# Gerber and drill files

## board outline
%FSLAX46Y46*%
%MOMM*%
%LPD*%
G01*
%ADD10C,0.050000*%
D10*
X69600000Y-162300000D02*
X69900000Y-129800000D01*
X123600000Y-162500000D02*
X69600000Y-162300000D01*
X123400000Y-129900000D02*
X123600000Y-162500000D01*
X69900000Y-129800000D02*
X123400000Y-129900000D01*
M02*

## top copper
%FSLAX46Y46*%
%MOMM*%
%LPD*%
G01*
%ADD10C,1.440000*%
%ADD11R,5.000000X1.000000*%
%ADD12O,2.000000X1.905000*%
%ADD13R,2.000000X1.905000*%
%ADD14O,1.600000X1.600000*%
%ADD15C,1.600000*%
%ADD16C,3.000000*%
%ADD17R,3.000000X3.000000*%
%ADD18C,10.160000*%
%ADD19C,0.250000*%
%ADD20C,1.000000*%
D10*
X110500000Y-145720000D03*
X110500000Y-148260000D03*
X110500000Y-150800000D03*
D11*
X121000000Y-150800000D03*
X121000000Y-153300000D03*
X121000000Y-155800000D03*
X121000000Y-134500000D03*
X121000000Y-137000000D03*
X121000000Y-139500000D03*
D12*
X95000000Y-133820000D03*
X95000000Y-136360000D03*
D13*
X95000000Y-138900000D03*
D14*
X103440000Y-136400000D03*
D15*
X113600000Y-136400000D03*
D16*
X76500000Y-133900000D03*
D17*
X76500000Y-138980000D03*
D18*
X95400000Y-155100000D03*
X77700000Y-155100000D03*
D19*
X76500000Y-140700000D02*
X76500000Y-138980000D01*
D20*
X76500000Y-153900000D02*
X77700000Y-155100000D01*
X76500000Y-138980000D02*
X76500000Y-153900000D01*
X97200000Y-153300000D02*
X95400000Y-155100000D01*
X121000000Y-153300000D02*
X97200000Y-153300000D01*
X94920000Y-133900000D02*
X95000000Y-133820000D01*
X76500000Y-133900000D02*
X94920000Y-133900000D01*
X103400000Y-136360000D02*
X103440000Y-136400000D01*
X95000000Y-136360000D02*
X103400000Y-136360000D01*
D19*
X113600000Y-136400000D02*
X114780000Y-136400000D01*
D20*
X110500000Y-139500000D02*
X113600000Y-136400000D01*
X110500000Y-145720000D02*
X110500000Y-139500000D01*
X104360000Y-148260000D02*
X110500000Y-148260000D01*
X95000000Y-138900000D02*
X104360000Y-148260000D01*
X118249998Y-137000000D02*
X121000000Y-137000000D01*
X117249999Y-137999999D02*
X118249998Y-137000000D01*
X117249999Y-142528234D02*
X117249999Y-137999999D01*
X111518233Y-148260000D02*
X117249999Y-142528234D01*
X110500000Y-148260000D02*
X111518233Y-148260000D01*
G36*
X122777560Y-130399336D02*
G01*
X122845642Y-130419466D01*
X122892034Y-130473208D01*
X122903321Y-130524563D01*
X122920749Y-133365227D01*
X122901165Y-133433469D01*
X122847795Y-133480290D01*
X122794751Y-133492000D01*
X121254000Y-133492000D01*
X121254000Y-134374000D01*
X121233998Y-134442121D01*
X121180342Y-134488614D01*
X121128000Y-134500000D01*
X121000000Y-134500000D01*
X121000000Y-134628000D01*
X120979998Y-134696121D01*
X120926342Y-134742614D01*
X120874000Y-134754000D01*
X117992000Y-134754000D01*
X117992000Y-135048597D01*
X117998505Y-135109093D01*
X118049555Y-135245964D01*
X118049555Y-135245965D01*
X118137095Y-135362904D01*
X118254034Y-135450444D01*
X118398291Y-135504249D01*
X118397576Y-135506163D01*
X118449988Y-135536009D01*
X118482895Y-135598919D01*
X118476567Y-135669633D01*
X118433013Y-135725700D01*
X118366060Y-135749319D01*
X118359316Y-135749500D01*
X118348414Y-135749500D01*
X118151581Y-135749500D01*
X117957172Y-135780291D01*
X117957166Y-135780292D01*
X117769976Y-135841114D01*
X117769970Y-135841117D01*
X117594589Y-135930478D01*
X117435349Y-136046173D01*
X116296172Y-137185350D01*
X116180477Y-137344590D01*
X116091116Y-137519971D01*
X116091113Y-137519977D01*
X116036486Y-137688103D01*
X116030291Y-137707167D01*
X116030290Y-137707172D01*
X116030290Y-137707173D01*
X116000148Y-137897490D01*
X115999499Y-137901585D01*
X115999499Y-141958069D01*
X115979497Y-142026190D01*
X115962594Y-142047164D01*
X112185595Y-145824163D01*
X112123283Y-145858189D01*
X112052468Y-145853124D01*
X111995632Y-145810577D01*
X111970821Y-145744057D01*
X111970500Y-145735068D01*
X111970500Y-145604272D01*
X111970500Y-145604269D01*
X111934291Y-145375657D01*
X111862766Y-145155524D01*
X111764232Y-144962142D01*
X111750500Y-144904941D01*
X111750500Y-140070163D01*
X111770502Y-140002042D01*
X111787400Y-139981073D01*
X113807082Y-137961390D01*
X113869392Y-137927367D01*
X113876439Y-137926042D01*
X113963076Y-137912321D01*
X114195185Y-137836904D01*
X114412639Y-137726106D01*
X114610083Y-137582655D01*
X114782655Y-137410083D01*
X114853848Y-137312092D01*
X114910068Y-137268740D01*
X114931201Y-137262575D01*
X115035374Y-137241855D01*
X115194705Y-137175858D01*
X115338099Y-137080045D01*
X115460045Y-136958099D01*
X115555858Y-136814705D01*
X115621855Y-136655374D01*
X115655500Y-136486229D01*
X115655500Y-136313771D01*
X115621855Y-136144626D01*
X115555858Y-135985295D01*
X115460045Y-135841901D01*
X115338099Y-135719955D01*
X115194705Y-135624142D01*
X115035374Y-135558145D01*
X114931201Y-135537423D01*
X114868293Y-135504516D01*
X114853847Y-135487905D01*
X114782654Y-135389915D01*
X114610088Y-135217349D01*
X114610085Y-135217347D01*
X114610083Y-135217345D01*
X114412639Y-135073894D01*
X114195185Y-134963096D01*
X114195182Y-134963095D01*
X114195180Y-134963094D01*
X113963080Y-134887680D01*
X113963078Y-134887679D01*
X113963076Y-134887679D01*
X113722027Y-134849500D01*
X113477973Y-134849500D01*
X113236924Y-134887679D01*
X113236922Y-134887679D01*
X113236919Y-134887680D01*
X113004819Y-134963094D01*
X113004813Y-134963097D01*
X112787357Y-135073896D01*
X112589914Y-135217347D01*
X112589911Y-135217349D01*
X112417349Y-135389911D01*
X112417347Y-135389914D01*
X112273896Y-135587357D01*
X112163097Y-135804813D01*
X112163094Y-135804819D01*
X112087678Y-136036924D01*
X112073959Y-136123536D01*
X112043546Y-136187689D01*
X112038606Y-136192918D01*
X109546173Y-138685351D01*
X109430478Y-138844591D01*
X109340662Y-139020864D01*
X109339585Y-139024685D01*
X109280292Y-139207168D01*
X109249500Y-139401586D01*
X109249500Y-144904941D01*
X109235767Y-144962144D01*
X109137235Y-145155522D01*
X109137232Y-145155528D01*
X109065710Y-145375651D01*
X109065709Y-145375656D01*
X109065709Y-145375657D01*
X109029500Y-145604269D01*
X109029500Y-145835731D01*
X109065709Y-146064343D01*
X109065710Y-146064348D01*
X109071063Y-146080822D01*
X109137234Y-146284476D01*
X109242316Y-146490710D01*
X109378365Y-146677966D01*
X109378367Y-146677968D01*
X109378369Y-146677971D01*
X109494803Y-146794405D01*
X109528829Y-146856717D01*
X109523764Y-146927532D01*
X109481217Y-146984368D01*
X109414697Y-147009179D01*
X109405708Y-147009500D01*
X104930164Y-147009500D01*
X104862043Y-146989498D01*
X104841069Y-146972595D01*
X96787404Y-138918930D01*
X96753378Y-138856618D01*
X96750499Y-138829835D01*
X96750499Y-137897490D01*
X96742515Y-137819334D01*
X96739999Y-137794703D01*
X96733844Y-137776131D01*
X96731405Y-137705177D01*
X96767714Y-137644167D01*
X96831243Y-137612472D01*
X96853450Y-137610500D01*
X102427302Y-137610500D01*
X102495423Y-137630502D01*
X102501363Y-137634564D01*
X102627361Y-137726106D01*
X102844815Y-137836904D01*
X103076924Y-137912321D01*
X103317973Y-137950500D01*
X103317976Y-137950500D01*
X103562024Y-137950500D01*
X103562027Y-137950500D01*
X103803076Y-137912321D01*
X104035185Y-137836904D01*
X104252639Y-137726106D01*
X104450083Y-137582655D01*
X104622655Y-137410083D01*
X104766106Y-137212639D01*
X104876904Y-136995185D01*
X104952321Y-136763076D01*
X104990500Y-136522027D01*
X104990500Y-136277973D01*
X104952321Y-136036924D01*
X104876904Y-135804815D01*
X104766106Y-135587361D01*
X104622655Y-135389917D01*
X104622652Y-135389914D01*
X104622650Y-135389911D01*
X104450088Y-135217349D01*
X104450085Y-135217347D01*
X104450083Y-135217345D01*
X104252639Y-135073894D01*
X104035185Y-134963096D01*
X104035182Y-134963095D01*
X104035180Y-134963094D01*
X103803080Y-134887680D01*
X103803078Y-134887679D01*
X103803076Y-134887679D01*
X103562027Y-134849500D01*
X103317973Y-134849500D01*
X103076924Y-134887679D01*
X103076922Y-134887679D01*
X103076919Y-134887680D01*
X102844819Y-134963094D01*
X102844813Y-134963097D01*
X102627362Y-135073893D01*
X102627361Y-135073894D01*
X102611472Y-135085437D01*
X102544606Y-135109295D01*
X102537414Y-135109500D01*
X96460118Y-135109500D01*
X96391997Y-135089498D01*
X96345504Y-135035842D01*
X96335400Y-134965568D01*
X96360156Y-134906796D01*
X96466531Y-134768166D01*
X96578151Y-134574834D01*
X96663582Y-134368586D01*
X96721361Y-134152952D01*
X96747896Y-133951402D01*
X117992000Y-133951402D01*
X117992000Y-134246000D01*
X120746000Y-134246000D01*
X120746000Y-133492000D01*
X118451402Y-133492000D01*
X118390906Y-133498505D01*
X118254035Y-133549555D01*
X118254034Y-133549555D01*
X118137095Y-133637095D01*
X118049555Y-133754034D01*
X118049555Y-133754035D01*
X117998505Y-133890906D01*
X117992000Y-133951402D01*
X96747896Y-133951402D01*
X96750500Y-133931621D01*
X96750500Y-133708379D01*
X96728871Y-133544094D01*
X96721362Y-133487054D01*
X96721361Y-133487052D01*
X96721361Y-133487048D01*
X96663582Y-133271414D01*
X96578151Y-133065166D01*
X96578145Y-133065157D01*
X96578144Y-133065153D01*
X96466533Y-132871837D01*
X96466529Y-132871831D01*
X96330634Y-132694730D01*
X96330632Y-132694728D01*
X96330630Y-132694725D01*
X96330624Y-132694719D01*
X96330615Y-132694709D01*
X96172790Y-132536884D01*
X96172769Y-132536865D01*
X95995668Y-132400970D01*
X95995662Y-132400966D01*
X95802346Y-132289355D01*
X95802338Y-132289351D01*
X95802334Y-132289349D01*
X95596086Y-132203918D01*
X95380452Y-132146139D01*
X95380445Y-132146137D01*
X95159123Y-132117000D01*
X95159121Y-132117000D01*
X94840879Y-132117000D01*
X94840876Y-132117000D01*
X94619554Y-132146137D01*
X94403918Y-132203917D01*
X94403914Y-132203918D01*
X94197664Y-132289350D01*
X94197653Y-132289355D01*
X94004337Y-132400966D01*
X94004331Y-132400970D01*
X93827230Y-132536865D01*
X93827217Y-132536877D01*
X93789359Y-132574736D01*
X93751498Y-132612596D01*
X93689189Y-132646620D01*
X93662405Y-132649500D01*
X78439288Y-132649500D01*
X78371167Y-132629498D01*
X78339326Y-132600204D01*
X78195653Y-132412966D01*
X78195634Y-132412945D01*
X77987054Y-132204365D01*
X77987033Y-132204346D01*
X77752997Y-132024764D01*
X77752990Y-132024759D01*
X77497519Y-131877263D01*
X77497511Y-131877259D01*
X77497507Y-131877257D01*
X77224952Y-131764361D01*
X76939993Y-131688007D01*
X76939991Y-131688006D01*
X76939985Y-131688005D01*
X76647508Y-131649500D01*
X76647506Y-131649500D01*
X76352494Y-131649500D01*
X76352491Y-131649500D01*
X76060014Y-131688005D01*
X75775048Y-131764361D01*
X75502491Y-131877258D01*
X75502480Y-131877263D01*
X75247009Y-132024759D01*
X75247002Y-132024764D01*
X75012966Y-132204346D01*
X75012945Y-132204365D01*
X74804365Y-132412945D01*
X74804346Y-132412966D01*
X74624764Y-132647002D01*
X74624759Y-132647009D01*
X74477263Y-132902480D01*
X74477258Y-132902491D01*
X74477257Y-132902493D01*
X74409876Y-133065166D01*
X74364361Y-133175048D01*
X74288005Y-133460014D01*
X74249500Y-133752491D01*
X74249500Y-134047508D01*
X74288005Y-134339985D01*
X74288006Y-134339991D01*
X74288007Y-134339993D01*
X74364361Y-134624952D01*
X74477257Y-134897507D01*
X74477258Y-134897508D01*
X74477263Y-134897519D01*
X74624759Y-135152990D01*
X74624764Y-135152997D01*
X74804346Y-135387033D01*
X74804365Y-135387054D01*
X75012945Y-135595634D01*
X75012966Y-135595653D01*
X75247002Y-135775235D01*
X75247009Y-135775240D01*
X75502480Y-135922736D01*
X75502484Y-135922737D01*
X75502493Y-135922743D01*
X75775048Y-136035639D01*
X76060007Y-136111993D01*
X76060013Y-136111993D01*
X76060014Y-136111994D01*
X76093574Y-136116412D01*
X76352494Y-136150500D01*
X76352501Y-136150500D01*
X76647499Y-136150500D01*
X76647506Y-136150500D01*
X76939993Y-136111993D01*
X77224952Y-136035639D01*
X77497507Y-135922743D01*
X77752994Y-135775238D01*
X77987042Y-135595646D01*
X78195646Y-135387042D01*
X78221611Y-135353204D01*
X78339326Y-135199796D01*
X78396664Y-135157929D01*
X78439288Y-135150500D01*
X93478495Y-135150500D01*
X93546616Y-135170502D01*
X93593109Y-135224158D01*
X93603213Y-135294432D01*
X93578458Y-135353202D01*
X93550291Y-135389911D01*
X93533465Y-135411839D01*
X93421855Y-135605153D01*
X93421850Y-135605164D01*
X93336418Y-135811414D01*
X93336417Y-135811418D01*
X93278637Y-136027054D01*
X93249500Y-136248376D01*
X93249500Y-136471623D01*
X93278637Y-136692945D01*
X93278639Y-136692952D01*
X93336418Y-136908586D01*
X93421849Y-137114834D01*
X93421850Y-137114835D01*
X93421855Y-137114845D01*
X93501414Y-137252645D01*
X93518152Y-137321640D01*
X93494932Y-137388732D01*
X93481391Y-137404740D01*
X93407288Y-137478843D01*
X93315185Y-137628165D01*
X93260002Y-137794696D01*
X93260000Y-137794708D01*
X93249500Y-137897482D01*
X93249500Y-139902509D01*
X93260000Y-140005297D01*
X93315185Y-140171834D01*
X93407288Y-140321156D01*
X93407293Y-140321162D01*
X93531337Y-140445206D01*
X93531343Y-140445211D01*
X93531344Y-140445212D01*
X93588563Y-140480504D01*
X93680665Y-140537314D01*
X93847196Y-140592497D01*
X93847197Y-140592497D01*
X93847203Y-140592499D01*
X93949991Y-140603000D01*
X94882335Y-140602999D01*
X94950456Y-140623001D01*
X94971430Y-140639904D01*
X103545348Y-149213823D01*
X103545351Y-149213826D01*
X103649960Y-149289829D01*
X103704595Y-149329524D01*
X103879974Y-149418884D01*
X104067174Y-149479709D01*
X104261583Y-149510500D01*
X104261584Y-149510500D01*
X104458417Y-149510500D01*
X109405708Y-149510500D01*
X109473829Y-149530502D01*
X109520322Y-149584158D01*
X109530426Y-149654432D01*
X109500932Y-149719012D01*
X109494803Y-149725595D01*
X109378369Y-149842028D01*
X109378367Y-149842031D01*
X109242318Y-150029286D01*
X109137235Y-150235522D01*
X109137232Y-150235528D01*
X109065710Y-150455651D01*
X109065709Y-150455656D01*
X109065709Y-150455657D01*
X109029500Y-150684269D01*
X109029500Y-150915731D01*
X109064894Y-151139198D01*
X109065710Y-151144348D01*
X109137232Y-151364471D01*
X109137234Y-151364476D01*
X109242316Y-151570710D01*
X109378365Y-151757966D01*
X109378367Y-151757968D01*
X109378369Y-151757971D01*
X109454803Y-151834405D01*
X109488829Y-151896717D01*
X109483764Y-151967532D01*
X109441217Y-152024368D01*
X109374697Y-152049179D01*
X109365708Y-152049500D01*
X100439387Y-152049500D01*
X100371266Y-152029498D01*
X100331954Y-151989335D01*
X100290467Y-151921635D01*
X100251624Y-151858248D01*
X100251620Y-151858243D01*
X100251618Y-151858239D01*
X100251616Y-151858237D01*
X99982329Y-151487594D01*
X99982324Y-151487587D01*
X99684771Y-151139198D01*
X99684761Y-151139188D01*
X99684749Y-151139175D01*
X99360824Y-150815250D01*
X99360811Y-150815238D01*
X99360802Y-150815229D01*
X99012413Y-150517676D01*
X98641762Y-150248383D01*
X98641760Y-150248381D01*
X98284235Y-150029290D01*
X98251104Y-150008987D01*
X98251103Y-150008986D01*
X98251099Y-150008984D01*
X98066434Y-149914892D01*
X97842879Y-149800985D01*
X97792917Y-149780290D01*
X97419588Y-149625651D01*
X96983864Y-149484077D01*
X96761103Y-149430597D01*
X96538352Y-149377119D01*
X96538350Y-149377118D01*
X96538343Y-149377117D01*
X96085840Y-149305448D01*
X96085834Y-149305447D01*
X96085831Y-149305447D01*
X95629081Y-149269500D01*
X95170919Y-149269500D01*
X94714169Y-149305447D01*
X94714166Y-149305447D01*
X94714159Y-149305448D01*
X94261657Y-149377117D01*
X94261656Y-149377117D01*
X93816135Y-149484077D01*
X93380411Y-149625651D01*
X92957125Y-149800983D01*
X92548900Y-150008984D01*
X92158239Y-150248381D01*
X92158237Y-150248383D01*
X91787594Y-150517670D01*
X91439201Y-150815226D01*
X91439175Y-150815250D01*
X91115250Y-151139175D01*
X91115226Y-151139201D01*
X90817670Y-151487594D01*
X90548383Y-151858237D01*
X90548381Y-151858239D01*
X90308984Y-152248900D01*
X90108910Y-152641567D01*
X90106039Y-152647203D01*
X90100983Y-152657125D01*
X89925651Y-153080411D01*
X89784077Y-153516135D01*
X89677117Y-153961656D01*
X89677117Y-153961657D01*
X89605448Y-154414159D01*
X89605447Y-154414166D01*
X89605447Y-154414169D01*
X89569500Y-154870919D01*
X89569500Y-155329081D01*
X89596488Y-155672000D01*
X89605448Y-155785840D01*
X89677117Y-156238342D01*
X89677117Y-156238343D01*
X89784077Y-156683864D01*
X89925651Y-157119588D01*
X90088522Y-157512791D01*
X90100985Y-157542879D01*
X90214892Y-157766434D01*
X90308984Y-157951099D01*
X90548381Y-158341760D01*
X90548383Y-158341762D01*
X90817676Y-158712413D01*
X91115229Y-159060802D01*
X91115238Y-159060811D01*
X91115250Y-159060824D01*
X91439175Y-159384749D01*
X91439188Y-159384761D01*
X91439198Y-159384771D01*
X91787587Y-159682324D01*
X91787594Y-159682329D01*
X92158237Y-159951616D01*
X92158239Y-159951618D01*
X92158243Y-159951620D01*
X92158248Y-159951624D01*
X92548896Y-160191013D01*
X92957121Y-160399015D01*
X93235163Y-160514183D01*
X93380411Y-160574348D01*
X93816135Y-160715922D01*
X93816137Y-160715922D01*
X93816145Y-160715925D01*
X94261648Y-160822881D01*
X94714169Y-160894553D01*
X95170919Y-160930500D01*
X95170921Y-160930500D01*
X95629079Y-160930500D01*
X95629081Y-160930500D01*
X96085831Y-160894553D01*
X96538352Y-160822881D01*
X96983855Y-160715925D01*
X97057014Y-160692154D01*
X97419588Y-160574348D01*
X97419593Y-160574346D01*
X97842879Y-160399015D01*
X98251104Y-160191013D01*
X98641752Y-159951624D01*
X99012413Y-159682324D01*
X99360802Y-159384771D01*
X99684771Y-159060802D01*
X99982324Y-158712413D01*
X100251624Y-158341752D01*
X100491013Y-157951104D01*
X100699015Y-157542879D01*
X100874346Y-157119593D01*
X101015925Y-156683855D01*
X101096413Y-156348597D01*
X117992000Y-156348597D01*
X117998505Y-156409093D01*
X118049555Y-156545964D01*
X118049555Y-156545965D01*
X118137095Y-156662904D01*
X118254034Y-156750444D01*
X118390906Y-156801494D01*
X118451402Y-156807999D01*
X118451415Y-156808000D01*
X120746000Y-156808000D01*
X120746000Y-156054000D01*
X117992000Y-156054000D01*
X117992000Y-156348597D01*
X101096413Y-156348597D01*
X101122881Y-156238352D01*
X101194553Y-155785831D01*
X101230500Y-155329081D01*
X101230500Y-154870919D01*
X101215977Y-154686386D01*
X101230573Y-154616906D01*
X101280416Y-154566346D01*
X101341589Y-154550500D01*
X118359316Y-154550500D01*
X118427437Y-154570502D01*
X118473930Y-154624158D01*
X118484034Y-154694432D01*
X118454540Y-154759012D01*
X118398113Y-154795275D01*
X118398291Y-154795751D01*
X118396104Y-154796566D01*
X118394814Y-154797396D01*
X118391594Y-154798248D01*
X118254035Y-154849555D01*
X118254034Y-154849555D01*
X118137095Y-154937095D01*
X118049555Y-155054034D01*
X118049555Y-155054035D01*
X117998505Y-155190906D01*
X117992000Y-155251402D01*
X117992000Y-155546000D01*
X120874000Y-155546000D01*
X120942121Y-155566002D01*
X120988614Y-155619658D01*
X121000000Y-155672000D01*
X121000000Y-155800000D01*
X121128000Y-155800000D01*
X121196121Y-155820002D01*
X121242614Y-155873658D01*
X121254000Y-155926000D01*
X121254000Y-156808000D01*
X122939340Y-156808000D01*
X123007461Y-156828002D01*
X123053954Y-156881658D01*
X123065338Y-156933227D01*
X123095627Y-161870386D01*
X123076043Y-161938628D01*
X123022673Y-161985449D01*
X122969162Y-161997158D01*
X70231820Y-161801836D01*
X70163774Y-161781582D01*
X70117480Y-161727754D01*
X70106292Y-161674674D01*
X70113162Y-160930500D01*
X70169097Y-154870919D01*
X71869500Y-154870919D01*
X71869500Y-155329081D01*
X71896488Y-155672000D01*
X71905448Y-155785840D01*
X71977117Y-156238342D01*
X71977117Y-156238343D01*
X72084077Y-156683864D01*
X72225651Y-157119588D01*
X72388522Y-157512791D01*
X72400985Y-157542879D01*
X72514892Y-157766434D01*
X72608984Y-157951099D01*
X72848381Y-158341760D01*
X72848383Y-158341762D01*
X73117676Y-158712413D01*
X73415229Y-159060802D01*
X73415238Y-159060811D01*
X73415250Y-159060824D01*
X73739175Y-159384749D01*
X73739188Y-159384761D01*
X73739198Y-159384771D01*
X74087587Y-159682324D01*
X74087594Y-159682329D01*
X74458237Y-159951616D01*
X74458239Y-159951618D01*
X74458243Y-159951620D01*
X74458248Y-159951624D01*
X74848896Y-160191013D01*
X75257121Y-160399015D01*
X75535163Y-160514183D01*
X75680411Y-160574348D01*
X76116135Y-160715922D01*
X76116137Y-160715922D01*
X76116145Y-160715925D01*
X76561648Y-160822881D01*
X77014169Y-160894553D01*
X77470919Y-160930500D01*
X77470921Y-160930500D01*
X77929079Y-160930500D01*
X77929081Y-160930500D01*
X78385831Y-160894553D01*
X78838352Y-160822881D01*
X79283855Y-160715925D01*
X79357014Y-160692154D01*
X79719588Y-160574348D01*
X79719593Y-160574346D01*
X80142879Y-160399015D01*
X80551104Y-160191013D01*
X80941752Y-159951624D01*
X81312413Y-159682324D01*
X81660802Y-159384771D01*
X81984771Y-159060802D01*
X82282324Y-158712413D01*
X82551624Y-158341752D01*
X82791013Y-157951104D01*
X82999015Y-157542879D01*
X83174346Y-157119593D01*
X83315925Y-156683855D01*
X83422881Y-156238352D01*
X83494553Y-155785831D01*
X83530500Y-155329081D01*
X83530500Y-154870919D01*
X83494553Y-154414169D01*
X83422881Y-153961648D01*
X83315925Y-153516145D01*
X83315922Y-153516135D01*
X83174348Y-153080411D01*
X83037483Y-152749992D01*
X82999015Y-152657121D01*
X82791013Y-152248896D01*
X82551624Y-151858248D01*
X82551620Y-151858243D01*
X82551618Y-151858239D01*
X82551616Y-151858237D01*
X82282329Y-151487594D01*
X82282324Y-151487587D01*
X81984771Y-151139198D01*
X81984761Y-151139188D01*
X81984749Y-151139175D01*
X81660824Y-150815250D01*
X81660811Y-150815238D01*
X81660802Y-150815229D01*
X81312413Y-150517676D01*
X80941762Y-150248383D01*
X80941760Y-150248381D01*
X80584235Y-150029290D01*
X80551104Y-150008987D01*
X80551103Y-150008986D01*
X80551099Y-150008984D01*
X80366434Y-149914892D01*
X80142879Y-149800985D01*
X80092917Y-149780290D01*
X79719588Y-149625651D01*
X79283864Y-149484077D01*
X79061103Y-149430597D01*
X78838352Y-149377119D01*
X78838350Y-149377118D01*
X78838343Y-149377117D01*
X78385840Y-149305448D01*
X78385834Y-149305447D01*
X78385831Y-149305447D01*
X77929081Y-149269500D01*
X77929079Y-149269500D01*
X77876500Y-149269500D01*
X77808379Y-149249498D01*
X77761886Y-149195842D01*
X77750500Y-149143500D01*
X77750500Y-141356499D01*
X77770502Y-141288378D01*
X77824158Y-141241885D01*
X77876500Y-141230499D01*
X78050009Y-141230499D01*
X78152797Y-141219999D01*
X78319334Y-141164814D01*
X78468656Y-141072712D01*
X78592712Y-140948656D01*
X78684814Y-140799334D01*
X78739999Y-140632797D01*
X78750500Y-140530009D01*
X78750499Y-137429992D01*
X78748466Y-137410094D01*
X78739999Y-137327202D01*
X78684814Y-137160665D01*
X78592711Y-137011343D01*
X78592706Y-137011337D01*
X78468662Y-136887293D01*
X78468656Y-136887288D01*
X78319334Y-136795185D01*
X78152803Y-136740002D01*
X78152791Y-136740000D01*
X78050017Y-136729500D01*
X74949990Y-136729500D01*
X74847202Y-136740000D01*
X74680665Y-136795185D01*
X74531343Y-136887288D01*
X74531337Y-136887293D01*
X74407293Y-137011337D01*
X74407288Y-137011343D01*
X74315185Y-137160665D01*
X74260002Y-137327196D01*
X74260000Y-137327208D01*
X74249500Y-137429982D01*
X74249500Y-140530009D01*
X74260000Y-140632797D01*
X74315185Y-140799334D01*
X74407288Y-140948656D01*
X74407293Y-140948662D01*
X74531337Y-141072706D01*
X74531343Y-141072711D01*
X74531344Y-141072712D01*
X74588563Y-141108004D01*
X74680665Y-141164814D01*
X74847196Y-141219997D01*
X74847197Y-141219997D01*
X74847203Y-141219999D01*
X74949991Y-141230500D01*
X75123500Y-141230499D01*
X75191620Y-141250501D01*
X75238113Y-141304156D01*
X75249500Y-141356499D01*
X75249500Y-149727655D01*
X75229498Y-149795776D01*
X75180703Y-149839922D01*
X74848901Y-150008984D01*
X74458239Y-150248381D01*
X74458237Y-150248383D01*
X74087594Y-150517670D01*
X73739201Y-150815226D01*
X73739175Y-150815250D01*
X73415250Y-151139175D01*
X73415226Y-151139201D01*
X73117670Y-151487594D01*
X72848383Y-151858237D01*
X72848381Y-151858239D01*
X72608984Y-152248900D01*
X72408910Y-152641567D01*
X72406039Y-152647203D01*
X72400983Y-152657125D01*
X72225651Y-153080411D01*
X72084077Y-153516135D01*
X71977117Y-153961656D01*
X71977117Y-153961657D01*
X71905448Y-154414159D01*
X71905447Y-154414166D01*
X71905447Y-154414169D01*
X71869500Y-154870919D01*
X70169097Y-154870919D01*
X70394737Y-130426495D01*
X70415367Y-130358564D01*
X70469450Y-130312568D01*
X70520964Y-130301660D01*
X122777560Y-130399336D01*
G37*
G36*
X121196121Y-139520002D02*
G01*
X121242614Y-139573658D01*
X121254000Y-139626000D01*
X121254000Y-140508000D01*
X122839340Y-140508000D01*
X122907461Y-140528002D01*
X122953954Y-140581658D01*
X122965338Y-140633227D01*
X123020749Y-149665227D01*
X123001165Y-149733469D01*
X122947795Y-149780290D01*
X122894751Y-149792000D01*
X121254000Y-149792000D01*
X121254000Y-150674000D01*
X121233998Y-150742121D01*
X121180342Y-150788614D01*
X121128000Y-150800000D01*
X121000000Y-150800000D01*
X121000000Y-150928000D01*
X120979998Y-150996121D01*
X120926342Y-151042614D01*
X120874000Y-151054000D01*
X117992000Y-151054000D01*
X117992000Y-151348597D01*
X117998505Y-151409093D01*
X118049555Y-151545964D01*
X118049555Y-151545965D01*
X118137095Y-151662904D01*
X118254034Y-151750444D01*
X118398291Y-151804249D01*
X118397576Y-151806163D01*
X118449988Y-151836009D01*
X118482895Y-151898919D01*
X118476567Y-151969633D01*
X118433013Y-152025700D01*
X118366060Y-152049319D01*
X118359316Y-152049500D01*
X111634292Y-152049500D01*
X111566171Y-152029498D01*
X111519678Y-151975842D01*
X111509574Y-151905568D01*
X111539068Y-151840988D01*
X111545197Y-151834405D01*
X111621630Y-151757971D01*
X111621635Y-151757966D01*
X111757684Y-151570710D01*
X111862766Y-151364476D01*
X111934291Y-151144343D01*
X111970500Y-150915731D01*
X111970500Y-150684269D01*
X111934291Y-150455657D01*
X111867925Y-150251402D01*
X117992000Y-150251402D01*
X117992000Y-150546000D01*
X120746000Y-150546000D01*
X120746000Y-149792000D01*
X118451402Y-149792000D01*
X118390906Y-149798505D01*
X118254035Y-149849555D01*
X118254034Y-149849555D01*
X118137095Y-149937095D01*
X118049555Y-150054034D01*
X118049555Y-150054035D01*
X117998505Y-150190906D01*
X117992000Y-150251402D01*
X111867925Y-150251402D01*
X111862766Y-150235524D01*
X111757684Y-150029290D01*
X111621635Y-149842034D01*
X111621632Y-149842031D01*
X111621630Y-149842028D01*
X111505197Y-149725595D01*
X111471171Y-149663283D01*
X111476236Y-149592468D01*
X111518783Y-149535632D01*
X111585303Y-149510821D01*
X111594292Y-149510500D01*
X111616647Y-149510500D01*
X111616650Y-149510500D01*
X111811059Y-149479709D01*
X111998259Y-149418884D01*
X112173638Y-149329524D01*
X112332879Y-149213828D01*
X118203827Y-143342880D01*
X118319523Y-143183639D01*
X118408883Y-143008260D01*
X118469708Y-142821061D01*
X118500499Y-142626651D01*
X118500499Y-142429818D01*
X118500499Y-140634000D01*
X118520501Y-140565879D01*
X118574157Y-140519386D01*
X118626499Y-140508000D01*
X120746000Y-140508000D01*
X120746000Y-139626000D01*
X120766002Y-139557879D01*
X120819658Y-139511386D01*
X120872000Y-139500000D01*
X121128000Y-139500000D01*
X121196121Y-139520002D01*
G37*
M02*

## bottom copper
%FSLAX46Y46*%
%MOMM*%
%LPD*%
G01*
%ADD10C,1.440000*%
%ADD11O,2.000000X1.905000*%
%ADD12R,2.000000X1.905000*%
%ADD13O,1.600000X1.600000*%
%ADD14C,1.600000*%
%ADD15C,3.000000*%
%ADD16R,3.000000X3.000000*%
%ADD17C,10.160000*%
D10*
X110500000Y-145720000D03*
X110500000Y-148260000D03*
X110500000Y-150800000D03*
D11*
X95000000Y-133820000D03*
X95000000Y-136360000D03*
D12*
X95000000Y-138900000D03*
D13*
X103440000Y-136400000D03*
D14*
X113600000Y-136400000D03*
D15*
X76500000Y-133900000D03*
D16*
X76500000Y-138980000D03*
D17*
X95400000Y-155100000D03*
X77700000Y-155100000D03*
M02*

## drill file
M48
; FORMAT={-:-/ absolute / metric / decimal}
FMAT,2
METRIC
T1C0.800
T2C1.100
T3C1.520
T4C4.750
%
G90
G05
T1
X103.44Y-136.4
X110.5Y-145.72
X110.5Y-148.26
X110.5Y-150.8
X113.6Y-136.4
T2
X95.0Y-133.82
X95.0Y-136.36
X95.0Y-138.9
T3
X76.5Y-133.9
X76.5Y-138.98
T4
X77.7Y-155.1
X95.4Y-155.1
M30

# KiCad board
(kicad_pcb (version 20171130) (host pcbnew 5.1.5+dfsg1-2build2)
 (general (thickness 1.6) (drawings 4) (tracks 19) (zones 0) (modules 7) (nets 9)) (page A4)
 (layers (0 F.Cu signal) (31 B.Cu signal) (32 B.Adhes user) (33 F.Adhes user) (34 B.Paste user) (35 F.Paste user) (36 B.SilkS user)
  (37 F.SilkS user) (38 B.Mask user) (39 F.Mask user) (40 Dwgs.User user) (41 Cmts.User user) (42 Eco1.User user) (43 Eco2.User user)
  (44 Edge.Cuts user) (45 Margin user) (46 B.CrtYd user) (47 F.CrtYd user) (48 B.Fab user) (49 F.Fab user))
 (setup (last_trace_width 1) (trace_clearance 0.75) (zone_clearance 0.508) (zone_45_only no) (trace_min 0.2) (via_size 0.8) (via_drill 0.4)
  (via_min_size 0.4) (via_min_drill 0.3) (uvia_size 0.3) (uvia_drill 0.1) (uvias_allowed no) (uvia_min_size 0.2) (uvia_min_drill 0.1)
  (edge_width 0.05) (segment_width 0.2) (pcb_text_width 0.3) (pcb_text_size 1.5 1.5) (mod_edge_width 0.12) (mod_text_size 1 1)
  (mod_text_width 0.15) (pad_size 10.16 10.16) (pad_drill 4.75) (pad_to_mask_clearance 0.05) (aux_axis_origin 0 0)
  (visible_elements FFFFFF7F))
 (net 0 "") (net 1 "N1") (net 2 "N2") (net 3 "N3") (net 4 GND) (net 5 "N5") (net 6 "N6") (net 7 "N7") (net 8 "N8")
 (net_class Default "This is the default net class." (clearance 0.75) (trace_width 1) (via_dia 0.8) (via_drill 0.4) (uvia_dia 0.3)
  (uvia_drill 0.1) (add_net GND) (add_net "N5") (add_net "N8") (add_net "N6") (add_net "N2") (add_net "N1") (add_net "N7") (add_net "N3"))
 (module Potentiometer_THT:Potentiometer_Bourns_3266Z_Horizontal (layer F.Cu) (at 110.5 150.8 270)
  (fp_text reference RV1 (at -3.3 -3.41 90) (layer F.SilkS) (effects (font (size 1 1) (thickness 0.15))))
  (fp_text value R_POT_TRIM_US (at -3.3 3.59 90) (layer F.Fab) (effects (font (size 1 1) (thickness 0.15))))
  (pad 3 thru_hole circle (at -5.08 0 270) (size 1.44 1.44) (drill 0.8) (layers *.Cu *.Mask) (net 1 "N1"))
  (pad 2 thru_hole circle (at -2.54 0 270) (size 1.44 1.44) (drill 0.8) (layers *.Cu *.Mask) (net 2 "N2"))
  (pad 1 thru_hole circle (at 0 0 270) (size 1.44 1.44) (drill 0.8) (layers *.Cu *.Mask) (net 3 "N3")))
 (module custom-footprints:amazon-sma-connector (layer F.Cu) (at 124 158.8 180)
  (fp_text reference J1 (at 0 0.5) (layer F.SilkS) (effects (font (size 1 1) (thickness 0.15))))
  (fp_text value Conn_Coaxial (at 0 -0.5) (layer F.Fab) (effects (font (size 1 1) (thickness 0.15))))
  (pad 2 connect rect (at 3 8 180) (size 5 1) (layers F.Cu F.Mask) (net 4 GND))
  (pad 1 connect rect (at 3 5.5 180) (size 5 1) (layers F.Cu F.Mask) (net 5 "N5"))
  (pad 2 connect rect (at 3 3 180) (size 5 1) (layers F.Cu F.Mask) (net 4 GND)))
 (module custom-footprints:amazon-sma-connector (layer F.Cu) (at 124 142.5 180)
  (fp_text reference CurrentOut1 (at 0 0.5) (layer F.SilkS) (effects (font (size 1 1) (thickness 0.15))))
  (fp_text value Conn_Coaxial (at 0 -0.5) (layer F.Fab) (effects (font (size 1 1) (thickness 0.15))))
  (pad 2 connect rect (at 3 8 180) (size 5 1) (layers F.Cu F.Mask) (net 4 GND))
  (pad 1 connect rect (at 3 5.5 180) (size 5 1) (layers F.Cu F.Mask) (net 2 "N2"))
  (pad 2 connect rect (at 3 3 180) (size 5 1) (layers F.Cu F.Mask) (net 4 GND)))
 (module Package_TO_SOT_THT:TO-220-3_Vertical (layer F.Cu) (at 95 138.9 90)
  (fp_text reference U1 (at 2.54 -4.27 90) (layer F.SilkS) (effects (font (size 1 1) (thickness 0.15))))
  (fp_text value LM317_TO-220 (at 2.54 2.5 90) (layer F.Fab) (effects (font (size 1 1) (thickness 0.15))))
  (pad 3 thru_hole oval (at 5.08 0 90) (size 1.905 2) (drill 1.1) (layers *.Cu *.Mask) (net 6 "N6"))
  (pad 2 thru_hole oval (at 2.54 0 90) (size 1.905 2) (drill 1.1) (layers *.Cu *.Mask) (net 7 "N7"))
  (pad 1 thru_hole rect (at 0 0 90) (size 1.905 2) (drill 1.1) (layers *.Cu *.Mask) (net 2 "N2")))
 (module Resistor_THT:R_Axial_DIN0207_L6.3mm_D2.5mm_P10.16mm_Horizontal (layer F.Cu) (at 113.6 136.4 180)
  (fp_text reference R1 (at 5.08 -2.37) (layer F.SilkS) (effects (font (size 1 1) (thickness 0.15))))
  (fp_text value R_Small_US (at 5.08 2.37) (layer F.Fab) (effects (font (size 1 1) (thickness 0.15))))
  (pad 2 thru_hole oval (at 10.16 0 180) (size 1.6 1.6) (drill 0.8) (layers *.Cu *.Mask) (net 7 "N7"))
  (pad 1 thru_hole circle (at 0 0 180) (size 1.6 1.6) (drill 0.8) (layers *.Cu *.Mask) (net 1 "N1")))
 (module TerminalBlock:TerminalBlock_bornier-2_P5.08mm (layer F.Cu) (at 76.5 138.98 90)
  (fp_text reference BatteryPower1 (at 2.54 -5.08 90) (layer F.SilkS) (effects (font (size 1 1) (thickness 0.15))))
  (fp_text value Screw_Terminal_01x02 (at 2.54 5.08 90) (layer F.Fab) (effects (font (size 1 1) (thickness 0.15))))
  (pad 2 thru_hole circle (at 5.08 0 90) (size 3 3) (drill 1.52) (layers *.Cu *.Mask) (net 6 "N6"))
  (pad 1 thru_hole rect (at 0 0 90) (size 3 3) (drill 1.52) (layers *.Cu *.Mask) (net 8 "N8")))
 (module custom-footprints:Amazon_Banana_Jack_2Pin (layer F.Cu) (at 95.4 155.1 180)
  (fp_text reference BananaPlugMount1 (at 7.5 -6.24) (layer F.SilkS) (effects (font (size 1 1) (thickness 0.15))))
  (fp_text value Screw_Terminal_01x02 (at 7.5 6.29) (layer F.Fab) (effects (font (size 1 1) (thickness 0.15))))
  (pad 1 thru_hole circle (at 0 0 180) (size 10.16 10.16) (drill 4.75) (layers *.Cu *.Mask) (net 5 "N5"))
  (pad 2 thru_hole circle (at 17.7 0 180) (size 10.16 10.16) (drill 4.75) (layers *.Cu *.Mask) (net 8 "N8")))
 (gr_line (start 69.6 162.3) (end 69.9 129.8) (layer Edge.Cuts) (width 0.05))
 (gr_line (start 123.6 162.5) (end 69.6 162.3) (layer Edge.Cuts) (width 0.05))
 (gr_line (start 123.4 129.9) (end 123.6 162.5) (layer Edge.Cuts) (width 0.05))
 (gr_line (start 69.9 129.8) (end 123.4 129.9) (layer Edge.Cuts) (width 0.05))
 (segment (start 76.5 140.7) (end 76.5 138.98) (width 0.25) (layer F.Cu) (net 8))
 (segment (start 76.5 153.9) (end 77.7 155.1) (width 1) (layer F.Cu) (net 8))
 (segment (start 76.5 138.98) (end 76.5 153.9) (width 1) (layer F.Cu) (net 8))
 (segment (start 97.2 153.3) (end 95.4 155.1) (width 1) (layer F.Cu) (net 5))
 (segment (start 121 153.3) (end 97.2 153.3) (width 1) (layer F.Cu) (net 5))
 (segment (start 94.92 133.9) (end 95 133.82) (width 1) (layer F.Cu) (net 6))
 (segment (start 76.5 133.9) (end 94.92 133.9) (width 1) (layer F.Cu) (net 6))
 (segment (start 103.4 136.36) (end 103.44 136.4) (width 1) (layer F.Cu) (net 7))
 (segment (start 95 136.36) (end 103.4 136.36) (width 1) (layer F.Cu) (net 7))
 (segment (start 113.6 136.4) (end 114.78 136.4) (width 0.25) (layer F.Cu) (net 1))
 (segment (start 110.5 139.5) (end 113.6 136.4) (width 1) (layer F.Cu) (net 1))
 (segment (start 110.5 145.72) (end 110.5 139.5) (width 1) (layer F.Cu) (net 1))
 (segment (start 104.36 148.26) (end 110.5 148.26) (width 1) (layer F.Cu) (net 2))
 (segment (start 95 138.9) (end 104.36 148.26) (width 1) (layer F.Cu) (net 2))
 (segment (start 118.249998 137) (end 121 137) (width 1) (layer F.Cu) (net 2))
 (segment (start 117.249999 137.999999) (end 118.249998 137) (width 1) (layer F.Cu) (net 2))
 (segment (start 117.249999 142.528234) (end 117.249999 137.999999) (width 1) (layer F.Cu) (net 2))
 (segment (start 111.518233 148.26) (end 117.249999 142.528234) (width 1) (layer F.Cu) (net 2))
 (segment (start 110.5 148.26) (end 111.518233 148.26) (width 1) (layer F.Cu) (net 2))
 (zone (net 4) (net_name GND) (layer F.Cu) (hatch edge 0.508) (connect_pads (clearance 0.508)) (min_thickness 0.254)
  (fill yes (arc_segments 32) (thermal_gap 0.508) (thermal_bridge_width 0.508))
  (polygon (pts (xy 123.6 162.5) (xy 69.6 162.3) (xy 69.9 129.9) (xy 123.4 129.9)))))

